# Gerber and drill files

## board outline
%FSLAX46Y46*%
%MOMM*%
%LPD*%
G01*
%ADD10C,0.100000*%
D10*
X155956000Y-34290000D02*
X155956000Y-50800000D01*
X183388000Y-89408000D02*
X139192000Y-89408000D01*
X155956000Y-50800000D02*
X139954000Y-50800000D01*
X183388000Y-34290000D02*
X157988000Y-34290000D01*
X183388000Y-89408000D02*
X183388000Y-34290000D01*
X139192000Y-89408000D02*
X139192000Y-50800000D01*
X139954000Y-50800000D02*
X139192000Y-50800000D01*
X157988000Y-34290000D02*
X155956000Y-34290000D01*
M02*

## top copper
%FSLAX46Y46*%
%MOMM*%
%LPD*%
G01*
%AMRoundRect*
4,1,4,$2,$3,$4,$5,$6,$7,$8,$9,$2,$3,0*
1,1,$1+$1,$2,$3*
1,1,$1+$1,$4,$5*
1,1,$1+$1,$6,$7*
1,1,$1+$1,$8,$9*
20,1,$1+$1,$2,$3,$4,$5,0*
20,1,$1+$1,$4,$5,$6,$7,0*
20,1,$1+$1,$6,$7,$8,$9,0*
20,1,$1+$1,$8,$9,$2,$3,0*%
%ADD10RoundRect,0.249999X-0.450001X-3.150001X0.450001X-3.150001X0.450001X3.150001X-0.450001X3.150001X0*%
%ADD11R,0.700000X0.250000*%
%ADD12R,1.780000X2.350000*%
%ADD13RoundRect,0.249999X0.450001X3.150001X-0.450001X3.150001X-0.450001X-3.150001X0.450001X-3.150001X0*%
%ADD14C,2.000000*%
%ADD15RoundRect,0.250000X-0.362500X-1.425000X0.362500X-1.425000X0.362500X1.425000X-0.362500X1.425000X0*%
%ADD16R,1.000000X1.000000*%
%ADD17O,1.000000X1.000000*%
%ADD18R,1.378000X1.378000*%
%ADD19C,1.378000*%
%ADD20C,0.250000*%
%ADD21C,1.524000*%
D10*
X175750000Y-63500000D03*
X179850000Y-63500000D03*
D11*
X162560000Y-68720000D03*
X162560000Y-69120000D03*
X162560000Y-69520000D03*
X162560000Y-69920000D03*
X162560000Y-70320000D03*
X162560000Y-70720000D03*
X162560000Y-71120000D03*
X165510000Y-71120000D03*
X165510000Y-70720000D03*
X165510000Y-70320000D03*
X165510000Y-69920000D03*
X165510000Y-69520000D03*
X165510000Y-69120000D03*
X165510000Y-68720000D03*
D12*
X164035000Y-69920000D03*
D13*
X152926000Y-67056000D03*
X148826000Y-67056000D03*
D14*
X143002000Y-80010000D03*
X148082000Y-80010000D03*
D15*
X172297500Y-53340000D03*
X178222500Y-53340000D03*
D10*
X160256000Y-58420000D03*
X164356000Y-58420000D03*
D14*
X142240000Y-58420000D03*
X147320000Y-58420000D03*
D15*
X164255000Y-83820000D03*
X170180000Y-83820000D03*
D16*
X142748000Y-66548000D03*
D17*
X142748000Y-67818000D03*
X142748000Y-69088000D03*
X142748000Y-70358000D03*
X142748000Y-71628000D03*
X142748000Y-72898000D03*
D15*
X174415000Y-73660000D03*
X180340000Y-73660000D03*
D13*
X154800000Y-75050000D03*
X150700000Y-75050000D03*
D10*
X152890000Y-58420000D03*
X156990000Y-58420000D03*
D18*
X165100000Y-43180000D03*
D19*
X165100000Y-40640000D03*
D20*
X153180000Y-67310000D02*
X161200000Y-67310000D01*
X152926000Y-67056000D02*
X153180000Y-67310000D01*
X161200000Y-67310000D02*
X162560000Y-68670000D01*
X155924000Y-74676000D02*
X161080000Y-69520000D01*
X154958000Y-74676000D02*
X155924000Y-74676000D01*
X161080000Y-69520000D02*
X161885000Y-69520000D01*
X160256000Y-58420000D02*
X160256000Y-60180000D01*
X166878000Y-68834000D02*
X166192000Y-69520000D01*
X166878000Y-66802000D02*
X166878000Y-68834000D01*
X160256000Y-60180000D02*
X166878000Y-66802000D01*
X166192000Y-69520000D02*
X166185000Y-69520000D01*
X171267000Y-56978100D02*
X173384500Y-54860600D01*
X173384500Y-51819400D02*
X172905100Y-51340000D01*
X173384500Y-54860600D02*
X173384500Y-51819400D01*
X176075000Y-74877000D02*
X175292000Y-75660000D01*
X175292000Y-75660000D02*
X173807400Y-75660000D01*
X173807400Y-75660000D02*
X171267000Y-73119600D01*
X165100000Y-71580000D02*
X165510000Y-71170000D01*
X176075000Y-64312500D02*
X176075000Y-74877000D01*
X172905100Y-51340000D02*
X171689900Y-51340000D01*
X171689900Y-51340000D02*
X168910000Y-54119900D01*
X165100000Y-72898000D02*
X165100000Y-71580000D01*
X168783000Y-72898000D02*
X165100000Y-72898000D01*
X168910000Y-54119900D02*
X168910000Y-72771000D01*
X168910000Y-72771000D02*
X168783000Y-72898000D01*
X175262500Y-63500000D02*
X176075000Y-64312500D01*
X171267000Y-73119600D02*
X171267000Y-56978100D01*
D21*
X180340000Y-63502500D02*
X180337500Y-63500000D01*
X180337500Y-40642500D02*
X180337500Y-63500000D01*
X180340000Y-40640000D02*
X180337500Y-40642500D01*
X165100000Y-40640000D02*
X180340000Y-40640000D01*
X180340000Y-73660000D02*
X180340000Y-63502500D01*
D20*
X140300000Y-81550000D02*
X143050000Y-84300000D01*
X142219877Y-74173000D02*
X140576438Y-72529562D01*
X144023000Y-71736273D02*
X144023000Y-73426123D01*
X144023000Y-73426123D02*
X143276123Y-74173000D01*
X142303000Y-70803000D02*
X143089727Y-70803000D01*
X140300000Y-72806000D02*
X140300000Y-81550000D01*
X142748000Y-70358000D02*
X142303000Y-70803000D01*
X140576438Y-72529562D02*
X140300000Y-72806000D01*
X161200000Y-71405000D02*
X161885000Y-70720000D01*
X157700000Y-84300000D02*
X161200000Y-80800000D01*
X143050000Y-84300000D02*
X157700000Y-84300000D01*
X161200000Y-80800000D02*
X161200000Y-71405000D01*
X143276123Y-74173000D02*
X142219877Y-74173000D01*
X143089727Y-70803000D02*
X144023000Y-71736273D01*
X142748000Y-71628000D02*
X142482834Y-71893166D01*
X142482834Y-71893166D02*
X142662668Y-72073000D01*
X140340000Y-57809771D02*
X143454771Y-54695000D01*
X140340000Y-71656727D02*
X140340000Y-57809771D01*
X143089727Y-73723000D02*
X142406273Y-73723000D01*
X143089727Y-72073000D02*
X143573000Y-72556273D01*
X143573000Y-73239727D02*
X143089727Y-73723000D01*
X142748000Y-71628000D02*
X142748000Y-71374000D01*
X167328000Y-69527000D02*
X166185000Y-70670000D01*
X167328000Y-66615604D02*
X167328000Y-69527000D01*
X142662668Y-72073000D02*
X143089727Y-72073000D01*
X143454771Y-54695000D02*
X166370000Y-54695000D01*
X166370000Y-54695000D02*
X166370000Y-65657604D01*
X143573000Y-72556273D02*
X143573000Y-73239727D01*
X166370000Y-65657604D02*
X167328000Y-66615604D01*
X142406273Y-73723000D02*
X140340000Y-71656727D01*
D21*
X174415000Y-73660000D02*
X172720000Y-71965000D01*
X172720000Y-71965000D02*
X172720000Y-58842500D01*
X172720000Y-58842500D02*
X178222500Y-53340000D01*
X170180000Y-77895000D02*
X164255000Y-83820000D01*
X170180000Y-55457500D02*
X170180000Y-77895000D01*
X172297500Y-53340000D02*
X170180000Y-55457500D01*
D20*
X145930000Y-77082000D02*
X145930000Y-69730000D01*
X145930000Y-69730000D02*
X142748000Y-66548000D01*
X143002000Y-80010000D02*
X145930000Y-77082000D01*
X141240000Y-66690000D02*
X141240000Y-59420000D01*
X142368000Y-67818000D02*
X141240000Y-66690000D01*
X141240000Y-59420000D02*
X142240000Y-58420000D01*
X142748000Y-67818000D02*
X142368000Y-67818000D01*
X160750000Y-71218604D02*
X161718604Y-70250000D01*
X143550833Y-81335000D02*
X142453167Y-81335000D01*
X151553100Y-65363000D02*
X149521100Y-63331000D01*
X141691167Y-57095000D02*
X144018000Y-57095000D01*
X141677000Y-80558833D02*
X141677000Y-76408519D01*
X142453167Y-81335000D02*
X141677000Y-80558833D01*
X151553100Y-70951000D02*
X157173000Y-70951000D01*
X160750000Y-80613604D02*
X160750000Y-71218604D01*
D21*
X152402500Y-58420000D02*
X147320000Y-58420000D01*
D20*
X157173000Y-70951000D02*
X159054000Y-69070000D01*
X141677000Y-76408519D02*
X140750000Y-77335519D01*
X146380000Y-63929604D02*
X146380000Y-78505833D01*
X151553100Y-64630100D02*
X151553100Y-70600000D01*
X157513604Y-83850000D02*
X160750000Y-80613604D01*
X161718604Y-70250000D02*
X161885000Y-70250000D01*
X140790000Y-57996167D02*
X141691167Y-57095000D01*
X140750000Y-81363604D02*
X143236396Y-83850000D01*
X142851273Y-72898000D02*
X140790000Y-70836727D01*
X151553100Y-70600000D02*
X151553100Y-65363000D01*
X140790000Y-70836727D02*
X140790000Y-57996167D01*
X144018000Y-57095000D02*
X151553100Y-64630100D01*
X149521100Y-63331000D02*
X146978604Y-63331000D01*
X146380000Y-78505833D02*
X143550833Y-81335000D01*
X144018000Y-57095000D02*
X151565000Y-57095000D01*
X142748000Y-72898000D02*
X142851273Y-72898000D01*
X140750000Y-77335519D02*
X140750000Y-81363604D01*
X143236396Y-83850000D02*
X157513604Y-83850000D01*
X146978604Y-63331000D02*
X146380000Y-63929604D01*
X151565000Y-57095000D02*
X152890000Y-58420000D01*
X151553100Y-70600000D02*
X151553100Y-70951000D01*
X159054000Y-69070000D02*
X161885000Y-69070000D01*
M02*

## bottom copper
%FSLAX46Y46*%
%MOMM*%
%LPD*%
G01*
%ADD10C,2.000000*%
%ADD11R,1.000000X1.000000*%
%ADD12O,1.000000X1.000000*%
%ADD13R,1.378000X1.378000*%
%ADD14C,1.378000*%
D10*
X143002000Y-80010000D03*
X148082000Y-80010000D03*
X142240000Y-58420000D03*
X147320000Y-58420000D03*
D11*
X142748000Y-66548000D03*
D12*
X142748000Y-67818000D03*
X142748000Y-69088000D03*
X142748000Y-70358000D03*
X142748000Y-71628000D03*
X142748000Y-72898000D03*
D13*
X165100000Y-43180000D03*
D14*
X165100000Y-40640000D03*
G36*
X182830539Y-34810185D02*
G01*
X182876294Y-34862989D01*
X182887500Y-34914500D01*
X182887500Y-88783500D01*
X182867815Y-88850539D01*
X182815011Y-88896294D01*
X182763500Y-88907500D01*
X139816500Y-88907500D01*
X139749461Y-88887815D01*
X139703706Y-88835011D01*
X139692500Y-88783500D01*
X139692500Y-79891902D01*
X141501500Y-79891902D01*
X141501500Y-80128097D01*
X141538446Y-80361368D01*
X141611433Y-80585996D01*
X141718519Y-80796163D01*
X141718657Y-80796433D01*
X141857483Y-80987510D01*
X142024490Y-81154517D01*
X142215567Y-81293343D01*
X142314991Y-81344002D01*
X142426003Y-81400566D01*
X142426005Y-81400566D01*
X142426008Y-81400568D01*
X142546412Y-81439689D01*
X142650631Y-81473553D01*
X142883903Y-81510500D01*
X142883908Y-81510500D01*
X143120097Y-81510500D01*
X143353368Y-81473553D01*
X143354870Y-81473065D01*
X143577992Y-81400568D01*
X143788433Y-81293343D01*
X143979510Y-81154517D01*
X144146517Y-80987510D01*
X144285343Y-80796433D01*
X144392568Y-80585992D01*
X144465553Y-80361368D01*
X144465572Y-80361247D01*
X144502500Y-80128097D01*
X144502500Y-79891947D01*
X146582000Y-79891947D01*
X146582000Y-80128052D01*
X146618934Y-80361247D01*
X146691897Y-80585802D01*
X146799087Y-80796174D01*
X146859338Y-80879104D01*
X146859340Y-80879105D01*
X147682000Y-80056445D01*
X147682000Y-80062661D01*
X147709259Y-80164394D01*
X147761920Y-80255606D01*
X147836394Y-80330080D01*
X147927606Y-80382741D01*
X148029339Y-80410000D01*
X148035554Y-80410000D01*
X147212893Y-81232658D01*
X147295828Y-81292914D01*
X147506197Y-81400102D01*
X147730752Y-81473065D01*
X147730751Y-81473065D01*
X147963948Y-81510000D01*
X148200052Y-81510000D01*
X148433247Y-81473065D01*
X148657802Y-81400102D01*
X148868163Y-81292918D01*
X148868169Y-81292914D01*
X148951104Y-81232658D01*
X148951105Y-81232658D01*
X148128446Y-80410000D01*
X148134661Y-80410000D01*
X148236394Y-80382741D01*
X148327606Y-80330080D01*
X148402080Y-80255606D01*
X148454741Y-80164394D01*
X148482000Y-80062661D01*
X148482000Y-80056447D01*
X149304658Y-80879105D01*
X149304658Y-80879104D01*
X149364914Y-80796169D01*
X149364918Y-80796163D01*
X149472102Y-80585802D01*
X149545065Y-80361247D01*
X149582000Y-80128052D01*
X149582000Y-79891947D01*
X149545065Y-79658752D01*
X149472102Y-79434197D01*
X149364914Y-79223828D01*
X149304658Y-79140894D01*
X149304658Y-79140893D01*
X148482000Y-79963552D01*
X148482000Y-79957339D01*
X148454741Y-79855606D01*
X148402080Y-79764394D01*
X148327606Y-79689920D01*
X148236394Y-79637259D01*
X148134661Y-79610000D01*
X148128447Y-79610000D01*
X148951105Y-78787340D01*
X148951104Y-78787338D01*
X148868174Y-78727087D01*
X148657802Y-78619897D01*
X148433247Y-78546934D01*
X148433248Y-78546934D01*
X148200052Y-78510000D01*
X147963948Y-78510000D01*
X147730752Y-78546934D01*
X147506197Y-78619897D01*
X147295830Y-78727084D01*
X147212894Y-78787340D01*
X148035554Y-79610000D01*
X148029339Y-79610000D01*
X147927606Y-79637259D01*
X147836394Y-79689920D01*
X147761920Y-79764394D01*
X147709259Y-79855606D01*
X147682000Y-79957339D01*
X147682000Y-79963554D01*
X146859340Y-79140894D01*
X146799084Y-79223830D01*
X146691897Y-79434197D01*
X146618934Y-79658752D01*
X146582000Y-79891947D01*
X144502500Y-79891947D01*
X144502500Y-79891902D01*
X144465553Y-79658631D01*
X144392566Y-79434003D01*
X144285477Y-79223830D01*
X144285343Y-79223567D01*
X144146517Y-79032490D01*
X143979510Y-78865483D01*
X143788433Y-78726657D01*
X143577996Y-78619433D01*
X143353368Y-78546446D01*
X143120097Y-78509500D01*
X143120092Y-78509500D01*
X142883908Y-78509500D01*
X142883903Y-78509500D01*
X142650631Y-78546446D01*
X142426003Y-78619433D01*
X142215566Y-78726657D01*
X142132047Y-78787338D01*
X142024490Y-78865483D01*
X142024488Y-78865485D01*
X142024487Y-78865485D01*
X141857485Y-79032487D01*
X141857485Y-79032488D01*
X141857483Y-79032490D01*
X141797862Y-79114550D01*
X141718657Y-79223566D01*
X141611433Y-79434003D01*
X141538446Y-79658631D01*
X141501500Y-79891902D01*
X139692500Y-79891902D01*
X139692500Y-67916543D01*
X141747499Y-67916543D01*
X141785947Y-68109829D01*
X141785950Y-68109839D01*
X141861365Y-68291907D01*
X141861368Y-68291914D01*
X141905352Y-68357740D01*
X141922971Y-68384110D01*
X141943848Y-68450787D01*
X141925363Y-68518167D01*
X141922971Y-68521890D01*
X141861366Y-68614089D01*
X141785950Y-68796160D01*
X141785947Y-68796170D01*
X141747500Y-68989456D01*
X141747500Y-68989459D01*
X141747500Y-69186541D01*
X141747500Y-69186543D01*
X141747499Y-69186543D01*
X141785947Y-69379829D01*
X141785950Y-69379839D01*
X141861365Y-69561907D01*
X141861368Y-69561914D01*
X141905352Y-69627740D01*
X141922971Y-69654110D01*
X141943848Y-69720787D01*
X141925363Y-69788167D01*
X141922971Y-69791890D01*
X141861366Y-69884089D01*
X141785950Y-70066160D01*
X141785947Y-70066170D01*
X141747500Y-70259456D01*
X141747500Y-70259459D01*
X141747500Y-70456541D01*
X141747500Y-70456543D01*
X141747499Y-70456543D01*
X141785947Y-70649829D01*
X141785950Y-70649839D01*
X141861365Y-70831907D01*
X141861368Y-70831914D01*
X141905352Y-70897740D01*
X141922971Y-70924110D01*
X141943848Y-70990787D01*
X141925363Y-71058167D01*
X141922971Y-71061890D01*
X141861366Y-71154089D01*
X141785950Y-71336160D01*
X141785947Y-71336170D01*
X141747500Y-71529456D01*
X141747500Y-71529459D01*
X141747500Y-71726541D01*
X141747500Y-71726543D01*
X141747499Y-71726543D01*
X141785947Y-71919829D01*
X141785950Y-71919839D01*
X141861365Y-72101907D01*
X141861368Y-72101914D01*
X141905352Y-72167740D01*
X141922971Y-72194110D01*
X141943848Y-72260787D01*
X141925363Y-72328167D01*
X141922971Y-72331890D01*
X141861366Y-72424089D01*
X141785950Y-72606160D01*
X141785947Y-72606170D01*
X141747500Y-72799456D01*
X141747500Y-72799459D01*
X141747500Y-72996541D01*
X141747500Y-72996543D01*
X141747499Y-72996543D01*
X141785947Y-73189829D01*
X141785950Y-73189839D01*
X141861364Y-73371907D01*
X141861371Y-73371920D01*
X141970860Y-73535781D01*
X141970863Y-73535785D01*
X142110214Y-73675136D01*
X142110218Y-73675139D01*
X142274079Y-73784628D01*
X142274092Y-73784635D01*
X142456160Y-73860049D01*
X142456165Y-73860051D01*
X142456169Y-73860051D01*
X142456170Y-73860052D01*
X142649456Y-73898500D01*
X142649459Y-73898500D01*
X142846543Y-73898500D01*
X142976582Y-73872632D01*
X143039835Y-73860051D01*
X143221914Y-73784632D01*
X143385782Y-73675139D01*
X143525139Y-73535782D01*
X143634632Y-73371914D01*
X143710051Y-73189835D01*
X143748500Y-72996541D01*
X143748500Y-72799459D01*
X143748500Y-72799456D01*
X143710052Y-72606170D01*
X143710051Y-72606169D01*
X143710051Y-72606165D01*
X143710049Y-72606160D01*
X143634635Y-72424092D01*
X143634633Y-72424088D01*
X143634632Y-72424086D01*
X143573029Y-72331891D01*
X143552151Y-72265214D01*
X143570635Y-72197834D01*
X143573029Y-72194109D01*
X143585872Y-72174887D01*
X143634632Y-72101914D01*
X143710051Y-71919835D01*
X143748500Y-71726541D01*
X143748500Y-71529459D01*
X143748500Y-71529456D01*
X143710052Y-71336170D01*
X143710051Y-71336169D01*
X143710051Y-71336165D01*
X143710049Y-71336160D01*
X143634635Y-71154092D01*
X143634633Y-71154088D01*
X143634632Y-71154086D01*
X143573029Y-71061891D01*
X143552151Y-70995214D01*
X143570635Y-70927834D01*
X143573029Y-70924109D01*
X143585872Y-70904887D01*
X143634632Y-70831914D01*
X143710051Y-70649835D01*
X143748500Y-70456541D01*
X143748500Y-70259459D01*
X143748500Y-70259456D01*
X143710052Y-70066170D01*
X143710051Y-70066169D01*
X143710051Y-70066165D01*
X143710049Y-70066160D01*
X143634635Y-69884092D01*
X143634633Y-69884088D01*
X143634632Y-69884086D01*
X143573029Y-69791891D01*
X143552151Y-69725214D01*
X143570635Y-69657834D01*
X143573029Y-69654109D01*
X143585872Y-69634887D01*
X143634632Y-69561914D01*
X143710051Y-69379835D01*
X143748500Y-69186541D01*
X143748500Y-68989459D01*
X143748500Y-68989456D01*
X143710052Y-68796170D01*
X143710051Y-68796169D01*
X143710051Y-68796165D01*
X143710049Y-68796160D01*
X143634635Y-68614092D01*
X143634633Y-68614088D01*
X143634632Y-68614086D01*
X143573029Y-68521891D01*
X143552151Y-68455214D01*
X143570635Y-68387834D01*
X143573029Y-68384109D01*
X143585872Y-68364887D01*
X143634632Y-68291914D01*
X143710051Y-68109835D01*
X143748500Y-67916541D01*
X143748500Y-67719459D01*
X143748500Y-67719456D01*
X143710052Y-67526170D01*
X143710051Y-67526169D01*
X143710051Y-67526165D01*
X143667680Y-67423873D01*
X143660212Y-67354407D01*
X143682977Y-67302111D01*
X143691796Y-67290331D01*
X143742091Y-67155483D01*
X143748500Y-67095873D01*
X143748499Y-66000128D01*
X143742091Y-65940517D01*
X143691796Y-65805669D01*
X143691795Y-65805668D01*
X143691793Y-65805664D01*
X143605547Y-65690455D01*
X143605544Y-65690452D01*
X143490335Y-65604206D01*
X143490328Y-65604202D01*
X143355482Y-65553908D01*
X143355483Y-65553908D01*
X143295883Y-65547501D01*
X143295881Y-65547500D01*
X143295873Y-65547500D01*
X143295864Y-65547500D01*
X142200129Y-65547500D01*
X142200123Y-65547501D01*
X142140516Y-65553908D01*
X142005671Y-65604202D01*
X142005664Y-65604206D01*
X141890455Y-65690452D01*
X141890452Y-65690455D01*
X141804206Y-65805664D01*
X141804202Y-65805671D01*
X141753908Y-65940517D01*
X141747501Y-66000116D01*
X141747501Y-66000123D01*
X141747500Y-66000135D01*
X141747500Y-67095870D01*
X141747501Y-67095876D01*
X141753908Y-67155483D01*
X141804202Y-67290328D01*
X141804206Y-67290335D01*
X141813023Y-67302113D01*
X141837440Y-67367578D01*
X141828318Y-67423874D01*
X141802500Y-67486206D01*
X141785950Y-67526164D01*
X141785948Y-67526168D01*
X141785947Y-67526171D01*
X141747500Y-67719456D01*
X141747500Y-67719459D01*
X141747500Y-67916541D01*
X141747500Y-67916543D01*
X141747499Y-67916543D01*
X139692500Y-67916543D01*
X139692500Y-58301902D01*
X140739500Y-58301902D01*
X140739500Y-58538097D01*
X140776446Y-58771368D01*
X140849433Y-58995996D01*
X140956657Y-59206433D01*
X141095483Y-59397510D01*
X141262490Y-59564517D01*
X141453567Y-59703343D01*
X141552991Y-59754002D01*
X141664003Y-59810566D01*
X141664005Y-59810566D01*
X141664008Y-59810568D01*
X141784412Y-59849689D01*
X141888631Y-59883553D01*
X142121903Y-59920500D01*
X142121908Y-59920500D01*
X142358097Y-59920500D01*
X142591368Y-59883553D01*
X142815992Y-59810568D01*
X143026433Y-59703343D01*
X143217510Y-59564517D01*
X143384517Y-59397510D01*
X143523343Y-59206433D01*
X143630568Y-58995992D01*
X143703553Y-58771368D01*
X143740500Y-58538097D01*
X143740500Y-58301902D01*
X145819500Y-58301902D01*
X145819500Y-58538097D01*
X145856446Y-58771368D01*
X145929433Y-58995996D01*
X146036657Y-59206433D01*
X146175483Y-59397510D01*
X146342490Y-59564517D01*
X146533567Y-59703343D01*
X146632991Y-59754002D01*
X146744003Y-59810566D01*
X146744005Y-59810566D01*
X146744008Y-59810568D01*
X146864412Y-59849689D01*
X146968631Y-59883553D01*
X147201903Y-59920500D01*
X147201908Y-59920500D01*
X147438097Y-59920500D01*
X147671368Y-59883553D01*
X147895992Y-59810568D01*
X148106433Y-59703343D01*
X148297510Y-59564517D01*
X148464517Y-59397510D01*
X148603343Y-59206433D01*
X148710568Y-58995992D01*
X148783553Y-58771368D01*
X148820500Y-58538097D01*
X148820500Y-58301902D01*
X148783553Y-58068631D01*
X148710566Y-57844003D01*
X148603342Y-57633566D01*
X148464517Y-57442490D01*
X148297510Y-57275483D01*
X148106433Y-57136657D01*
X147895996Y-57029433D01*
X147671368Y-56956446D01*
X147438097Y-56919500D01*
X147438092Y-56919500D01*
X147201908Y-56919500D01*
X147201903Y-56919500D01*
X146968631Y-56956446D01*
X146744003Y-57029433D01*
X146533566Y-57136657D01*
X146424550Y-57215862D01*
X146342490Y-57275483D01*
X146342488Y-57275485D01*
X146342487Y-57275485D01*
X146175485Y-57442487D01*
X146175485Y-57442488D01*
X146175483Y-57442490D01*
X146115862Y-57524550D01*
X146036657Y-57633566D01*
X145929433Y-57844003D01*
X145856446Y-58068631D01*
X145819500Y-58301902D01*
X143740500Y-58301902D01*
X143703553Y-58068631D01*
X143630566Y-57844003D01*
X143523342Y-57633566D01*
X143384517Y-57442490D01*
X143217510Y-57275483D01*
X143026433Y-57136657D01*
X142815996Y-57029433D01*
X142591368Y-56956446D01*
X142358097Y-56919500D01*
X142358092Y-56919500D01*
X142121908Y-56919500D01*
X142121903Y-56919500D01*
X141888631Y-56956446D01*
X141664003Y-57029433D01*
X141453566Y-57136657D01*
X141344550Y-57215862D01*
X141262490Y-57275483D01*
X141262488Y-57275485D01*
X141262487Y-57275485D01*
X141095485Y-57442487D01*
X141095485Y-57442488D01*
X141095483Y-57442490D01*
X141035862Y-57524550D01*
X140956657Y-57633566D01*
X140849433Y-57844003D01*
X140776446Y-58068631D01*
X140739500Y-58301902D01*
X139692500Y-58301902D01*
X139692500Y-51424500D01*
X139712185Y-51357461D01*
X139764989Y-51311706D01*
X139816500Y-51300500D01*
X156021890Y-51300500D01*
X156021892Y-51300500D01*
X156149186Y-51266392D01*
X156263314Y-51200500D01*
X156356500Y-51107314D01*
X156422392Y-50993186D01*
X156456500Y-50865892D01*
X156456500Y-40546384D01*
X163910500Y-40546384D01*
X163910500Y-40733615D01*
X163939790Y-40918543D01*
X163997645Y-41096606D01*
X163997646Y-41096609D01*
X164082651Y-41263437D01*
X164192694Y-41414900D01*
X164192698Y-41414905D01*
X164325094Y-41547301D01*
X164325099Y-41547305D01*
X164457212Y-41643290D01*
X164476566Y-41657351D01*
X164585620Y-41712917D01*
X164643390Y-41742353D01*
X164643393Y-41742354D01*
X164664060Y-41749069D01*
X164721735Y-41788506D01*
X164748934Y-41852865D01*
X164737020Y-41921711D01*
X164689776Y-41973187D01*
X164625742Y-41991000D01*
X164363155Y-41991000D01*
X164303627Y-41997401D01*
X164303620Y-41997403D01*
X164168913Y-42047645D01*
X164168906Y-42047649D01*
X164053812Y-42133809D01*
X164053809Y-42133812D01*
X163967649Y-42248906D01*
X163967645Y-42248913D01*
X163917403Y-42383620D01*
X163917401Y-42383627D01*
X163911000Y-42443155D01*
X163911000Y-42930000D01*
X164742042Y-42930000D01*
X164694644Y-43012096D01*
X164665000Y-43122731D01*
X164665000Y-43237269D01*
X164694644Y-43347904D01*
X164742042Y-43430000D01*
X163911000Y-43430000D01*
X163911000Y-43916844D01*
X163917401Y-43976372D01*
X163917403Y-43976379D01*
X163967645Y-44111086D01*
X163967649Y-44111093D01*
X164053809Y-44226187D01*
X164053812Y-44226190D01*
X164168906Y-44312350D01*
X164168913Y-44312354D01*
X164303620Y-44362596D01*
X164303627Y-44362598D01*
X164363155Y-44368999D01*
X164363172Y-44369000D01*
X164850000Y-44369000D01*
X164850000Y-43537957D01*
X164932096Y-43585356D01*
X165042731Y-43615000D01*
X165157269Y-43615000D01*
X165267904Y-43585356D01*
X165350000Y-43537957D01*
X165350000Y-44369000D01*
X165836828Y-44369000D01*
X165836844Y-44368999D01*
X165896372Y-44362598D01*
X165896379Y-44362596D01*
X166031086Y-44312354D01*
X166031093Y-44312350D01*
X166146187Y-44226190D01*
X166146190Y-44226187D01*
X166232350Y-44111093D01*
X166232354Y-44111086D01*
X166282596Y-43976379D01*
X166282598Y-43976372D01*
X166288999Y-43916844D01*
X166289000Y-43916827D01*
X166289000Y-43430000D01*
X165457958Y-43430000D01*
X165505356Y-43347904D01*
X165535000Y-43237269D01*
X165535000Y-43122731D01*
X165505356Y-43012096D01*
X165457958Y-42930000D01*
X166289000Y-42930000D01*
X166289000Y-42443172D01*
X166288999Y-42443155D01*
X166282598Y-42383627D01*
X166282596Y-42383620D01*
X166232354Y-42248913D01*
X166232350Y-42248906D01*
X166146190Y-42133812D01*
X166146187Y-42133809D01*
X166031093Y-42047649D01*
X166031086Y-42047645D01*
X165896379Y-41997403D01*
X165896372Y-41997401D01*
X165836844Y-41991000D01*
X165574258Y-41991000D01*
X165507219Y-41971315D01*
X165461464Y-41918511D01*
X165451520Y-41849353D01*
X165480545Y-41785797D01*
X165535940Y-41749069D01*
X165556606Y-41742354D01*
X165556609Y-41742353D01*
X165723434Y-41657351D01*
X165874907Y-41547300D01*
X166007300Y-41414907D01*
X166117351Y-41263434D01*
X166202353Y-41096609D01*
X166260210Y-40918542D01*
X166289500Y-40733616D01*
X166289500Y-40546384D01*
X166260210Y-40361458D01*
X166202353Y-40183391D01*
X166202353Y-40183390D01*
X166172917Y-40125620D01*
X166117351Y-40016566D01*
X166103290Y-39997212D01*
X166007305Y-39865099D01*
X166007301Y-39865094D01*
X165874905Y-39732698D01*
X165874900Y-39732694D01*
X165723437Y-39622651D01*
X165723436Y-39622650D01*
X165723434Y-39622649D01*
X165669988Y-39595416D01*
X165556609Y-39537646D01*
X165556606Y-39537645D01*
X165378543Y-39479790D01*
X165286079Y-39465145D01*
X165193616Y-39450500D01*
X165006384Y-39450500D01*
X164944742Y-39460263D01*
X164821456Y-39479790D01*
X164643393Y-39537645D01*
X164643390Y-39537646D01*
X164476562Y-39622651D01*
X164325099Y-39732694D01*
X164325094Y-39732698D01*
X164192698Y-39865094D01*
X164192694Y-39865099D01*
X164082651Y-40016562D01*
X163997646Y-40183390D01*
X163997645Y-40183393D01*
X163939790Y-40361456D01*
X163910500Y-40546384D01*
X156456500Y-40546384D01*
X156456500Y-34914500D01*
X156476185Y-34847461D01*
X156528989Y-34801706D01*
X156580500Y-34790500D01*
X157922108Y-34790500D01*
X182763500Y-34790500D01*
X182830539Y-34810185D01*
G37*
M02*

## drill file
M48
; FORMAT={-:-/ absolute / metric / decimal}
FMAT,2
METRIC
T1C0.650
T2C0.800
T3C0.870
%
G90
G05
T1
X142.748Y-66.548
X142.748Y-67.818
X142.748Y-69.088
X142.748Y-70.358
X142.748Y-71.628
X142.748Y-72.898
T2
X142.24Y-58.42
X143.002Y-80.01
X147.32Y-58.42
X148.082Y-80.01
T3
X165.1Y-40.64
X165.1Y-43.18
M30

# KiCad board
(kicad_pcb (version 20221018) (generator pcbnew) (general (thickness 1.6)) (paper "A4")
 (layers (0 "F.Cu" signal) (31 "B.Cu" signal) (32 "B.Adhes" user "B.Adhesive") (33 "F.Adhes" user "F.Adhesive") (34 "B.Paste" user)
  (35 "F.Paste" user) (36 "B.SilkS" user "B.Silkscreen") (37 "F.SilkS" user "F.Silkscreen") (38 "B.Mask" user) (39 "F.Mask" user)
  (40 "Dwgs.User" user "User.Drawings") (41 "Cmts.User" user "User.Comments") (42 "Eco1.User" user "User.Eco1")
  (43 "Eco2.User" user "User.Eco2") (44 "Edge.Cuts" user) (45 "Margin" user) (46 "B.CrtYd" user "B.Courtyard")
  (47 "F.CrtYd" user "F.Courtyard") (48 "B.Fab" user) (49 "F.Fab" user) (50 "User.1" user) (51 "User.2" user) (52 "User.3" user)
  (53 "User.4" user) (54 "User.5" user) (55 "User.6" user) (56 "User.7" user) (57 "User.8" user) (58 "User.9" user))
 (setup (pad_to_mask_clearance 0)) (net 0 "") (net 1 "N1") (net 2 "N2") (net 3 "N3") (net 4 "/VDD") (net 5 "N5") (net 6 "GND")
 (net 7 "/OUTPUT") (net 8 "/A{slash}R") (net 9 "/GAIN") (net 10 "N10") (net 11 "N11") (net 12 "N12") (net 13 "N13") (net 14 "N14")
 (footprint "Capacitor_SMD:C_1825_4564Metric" (layer "F.Cu") (at 177.8 63.5)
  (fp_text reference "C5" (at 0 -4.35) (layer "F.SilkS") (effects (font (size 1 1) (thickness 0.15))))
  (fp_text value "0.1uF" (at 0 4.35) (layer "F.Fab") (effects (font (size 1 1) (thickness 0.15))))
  (pad "1" smd roundrect (at -2.05 0) (size 1.4 6.8) (layers "F.Cu" "F.Paste" "F.Mask") (roundrect_rratio 0.178571) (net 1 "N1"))
  (pad "2" smd roundrect (at 2.05 0) (size 1.4 6.8) (layers "F.Cu" "F.Paste" "F.Mask") (roundrect_rratio 0.178571) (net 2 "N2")))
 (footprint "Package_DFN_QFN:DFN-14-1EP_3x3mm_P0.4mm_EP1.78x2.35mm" (layer "F.Cu") (at 164.035 69.92)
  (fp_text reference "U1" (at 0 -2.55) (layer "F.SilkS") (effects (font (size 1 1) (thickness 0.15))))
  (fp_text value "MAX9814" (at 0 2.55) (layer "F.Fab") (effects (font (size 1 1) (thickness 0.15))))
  (pad "" smd rect (at -0.445 -0.5875) (size 0.7 0.97) (layers "F.Paste"))
  (pad "" smd rect (at -0.445 0.5875) (size 0.7 0.97) (layers "F.Paste"))
  (pad "" smd rect (at 0.45 -0.5875) (size 0.7 0.97) (layers "F.Paste"))
  (pad "" smd rect (at 0.45 0.5875) (size 0.7 0.97) (layers "F.Paste"))
  (pad "1" smd rect (at -1.475 -1.2) (size 0.7 0.25) (layers "F.Cu" "F.Paste" "F.Mask") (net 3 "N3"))
  (pad "2" smd rect (at -1.475 -0.8) (size 0.7 0.25) (layers "F.Cu" "F.Paste" "F.Mask") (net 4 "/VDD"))
  (pad "3" smd rect (at -1.475 -0.4) (size 0.7 0.25) (layers "F.Cu" "F.Paste" "F.Mask") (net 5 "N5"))
  (pad "4" smd rect (at -1.475 0) (size 0.7 0.25) (layers "F.Cu" "F.Paste" "F.Mask") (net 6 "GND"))
  (pad "5" smd rect (at -1.475 0.4) (size 0.7 0.25) (layers "F.Cu" "F.Paste" "F.Mask") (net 4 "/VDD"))
  (pad "6" smd rect (at -1.475 0.8) (size 0.7 0.25) (layers "F.Cu" "F.Paste" "F.Mask") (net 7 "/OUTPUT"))
  (pad "7" smd rect (at -1.475 1.2) (size 0.7 0.25) (layers "F.Cu" "F.Paste" "F.Mask") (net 6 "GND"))
  (pad "8" smd rect (at 1.475 1.2) (size 0.7 0.25) (layers "F.Cu" "F.Paste" "F.Mask") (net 1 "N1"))
  (pad "9" smd rect (at 1.475 0.8) (size 0.7 0.25) (layers "F.Cu" "F.Paste" "F.Mask") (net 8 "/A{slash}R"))
  (pad "10" smd rect (at 1.475 0.4) (size 0.7 0.25) (layers "F.Cu" "F.Paste" "F.Mask") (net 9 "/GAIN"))
  (pad "11" smd rect (at 1.475 0) (size 0.7 0.25) (layers "F.Cu" "F.Paste" "F.Mask") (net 6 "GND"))
  (pad "12" smd rect (at 1.475 -0.4) (size 0.7 0.25) (layers "F.Cu" "F.Paste" "F.Mask") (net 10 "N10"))
  (pad "13" smd rect (at 1.475 -0.8) (size 0.7 0.25) (layers "F.Cu" "F.Paste" "F.Mask") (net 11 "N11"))
  (pad "14" smd rect (at 1.475 -1.2) (size 0.7 0.25) (layers "F.Cu" "F.Paste" "F.Mask") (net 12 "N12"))
  (pad "15" smd rect (at 0 0) (size 1.78 2.35) (layers "F.Cu" "F.Mask") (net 6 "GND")))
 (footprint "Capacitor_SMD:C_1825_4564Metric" (layer "F.Cu") (at 150.876 67.056 180)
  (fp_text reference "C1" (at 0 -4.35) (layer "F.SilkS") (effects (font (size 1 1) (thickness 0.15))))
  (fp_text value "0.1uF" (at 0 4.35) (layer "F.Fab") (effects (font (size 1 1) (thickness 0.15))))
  (pad "1" smd roundrect (at -2.05 0 180) (size 1.4 6.8) (layers "F.Cu" "F.Paste" "F.Mask") (roundrect_rratio 0.178571) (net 3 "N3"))
  (pad "2" smd roundrect (at 2.05 0 180) (size 1.4 6.8) (layers "F.Cu" "F.Paste" "F.Mask") (roundrect_rratio 0.178571) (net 6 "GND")))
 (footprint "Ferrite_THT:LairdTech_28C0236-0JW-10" (layer "F.Cu") (at 143.002 80.01)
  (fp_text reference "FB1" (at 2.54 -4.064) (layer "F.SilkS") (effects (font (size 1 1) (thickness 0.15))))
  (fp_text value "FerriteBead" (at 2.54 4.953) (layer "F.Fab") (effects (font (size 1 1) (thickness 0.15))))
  (pad "1" thru_hole circle (at 0 0) (size 2 2) (drill 0.8) (layers "*.Cu" "*.Mask") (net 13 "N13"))
  (pad "2" thru_hole circle (at 5.08 0) (size 2 2) (drill 0.8) (layers "*.Cu" "*.Mask") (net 6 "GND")))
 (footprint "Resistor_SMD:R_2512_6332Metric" (layer "F.Cu") (at 175.26 53.34)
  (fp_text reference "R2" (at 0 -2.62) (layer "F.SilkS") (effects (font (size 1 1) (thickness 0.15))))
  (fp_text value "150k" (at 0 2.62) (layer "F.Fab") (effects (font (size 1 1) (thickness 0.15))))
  (pad "1" smd roundrect (at -2.9625 0) (size 1.225 3.35) (layers "F.Cu" "F.Paste" "F.Mask") (roundrect_rratio 0.204082) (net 12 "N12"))
  (pad "2" smd roundrect (at 2.9625 0) (size 1.225 3.35) (layers "F.Cu" "F.Paste" "F.Mask") (roundrect_rratio 0.204082) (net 11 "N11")))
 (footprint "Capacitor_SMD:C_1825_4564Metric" (layer "F.Cu") (at 162.306 58.42)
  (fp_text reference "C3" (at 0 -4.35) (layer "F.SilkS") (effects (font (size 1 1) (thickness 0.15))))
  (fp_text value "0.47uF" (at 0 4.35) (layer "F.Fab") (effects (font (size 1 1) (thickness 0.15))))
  (pad "1" smd roundrect (at -2.05 0) (size 1.4 6.8) (layers "F.Cu" "F.Paste" "F.Mask") (roundrect_rratio 0.178571) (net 10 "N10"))
  (pad "2" smd roundrect (at 2.05 0) (size 1.4 6.8) (layers "F.Cu" "F.Paste" "F.Mask") (roundrect_rratio 0.178571) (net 6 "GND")))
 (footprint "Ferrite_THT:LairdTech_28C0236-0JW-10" (layer "F.Cu") (at 142.24 58.42)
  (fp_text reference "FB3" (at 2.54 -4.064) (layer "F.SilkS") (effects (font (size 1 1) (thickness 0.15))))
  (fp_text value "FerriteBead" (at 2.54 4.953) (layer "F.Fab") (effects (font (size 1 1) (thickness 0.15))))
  (pad "1" thru_hole circle (at 0 0) (size 2 2) (drill 0.8) (layers "*.Cu" "*.Mask") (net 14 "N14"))
  (pad "2" thru_hole circle (at 5.08 0) (size 2 2) (drill 0.8) (layers "*.Cu" "*.Mask") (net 4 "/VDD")))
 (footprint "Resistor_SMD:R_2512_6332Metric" (layer "F.Cu") (at 167.2175 83.82)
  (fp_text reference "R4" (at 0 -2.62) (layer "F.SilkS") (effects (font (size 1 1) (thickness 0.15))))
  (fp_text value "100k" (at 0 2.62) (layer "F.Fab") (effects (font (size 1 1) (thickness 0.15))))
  (pad "1" smd roundrect (at -2.9625 0) (size 1.225 3.35) (layers "F.Cu" "F.Paste" "F.Mask") (roundrect_rratio 0.204082) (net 12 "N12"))
  (pad "2" smd roundrect (at 2.9625 0) (size 1.225 3.35) (layers "F.Cu" "F.Paste" "F.Mask") (roundrect_rratio 0.204082) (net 6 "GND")))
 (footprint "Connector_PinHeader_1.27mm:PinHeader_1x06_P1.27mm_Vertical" (layer "F.Cu") (at 142.748 66.548)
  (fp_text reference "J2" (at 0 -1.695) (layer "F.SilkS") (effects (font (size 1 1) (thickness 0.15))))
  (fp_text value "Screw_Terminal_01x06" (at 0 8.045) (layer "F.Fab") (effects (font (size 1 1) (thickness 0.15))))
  (pad "1" thru_hole rect (at 0 0) (size 1 1) (drill 0.65) (layers "*.Cu" "*.Mask") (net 13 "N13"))
  (pad "2" thru_hole oval (at 0 1.27) (size 1 1) (drill 0.65) (layers "*.Cu" "*.Mask") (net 14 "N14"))
  (pad "3" thru_hole oval (at 0 2.54) (size 1 1) (drill 0.65) (layers "*.Cu" "*.Mask") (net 9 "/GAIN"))
  (pad "4" thru_hole oval (at 0 3.81) (size 1 1) (drill 0.65) (layers "*.Cu" "*.Mask") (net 7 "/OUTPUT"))
  (pad "5" thru_hole oval (at 0 5.08) (size 1 1) (drill 0.65) (layers "*.Cu" "*.Mask") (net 8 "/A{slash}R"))
  (pad "6" thru_hole oval (at 0 6.35) (size 1 1) (drill 0.65) (layers "*.Cu" "*.Mask") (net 4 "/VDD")))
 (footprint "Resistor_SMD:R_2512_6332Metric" (layer "F.Cu") (at 177.3775 73.66)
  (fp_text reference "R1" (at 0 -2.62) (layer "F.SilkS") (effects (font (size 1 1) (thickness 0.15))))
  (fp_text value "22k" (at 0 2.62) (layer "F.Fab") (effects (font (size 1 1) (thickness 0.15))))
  (pad "1" smd roundrect (at -2.9625 0) (size 1.225 3.35) (layers "F.Cu" "F.Paste" "F.Mask") (roundrect_rratio 0.204082) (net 11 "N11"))
  (pad "2" smd roundrect (at 2.9625 0) (size 1.225 3.35) (layers "F.Cu" "F.Paste" "F.Mask") (roundrect_rratio 0.204082) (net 2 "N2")))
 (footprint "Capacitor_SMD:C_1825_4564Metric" (layer "F.Cu") (at 152.75 75.05 180)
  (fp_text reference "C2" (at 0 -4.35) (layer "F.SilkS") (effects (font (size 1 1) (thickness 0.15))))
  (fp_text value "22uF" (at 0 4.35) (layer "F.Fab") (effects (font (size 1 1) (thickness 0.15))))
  (pad "1" smd roundrect (at -2.05 0 180) (size 1.4 6.8) (layers "F.Cu" "F.Paste" "F.Mask") (roundrect_rratio 0.178571) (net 5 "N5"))
  (pad "2" smd roundrect (at 2.05 0 180) (size 1.4 6.8) (layers "F.Cu" "F.Paste" "F.Mask") (roundrect_rratio 0.178571) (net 6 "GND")))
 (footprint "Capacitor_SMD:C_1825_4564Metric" (layer "F.Cu") (at 154.94 58.42)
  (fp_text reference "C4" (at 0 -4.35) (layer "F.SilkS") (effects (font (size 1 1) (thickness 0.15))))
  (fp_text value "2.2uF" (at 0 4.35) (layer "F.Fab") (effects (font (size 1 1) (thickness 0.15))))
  (pad "1" smd roundrect (at -2.05 0) (size 1.4 6.8) (layers "F.Cu" "F.Paste" "F.Mask") (roundrect_rratio 0.178571) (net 4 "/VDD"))
  (pad "2" smd roundrect (at 2.05 0) (size 1.4 6.8) (layers "F.Cu" "F.Paste" "F.Mask") (roundrect_rratio 0.178571) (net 6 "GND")))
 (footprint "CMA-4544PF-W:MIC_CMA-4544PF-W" (layer "F.Cu") (at 163.1 41.91)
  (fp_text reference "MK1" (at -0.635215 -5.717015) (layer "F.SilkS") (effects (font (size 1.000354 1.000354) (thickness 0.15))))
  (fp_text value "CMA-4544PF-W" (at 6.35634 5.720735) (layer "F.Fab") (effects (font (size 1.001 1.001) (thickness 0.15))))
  (pad "1" thru_hole rect (at 2 1.27) (size 1.378 1.378) (drill 0.87) (layers "*.Cu" "*.Mask") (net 6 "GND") (solder_mask_margin 0.102))
  (pad "2" thru_hole circle (at 2 -1.27) (size 1.378 1.378) (drill 0.87) (layers "*.Cu" "*.Mask") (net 2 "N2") (solder_mask_margin 0.102)))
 (gr_line (start 155.956 34.29) (end 155.956 50.8) (stroke (width 0.1) (type default)) (layer "Edge.Cuts"))
 (gr_line (start 183.388 89.408) (end 139.192 89.408) (stroke (width 0.1) (type default)) (layer "Edge.Cuts"))
 (gr_line (start 155.956 50.8) (end 139.954 50.8) (stroke (width 0.1) (type default)) (layer "Edge.Cuts"))
 (gr_line (start 183.388 34.29) (end 157.988 34.29) (stroke (width 0.1) (type default)) (layer "Edge.Cuts"))
 (gr_line (start 183.388 89.408) (end 183.388 34.29) (stroke (width 0.1) (type default)) (layer "Edge.Cuts"))
 (gr_line (start 139.192 89.408) (end 139.192 50.8) (stroke (width 0.1) (type default)) (layer "Edge.Cuts"))
 (gr_line (start 139.954 50.8) (end 139.192 50.8) (stroke (width 0.1) (type default)) (layer "Edge.Cuts"))
 (gr_line (start 157.988 34.29) (end 155.956 34.29) (stroke (width 0.1) (type default)) (layer "Edge.Cuts"))
 (segment (start 153.18 67.31) (end 161.2 67.31) (width 0.25) (layer "F.Cu") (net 3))
 (segment (start 152.926 67.056) (end 153.18 67.31) (width 0.25) (layer "F.Cu") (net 3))
 (segment (start 161.2 67.31) (end 162.56 68.67) (width 0.25) (layer "F.Cu") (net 3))
 (segment (start 155.924 74.676) (end 161.08 69.52) (width 0.25) (layer "F.Cu") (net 5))
 (segment (start 154.958 74.676) (end 155.924 74.676) (width 0.25) (layer "F.Cu") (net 5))
 (segment (start 161.08 69.52) (end 161.885 69.52) (width 0.25) (layer "F.Cu") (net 5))
 (segment (start 160.256 58.42) (end 160.256 60.18) (width 0.25) (layer "F.Cu") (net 10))
 (segment (start 166.878 68.834) (end 166.192 69.52) (width 0.25) (layer "F.Cu") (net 10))
 (segment (start 166.878 66.802) (end 166.878 68.834) (width 0.25) (layer "F.Cu") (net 10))
 (segment (start 160.256 60.18) (end 166.878 66.802) (width 0.25) (layer "F.Cu") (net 10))
 (segment (start 166.192 69.52) (end 166.185 69.52) (width 0.25) (layer "F.Cu") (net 10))
 (segment (start 171.267 56.9781) (end 173.3845 54.8606) (width 0.25) (layer "F.Cu") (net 1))
 (segment (start 173.3845 51.8194) (end 172.9051 51.34) (width 0.25) (layer "F.Cu") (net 1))
 (segment (start 173.3845 54.8606) (end 173.3845 51.8194) (width 0.25) (layer "F.Cu") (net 1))
 (segment (start 176.075 74.877) (end 175.292 75.66) (width 0.25) (layer "F.Cu") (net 1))
 (segment (start 175.292 75.66) (end 173.8074 75.66) (width 0.25) (layer "F.Cu") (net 1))
 (segment (start 173.8074 75.66) (end 171.267 73.1196) (width 0.25) (layer "F.Cu") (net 1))
 (segment (start 165.1 71.58) (end 165.51 71.17) (width 0.25) (layer "F.Cu") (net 1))
 (segment (start 176.075 64.3125) (end 176.075 74.877) (width 0.25) (layer "F.Cu") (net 1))
 (segment (start 172.9051 51.34) (end 171.6899 51.34) (width 0.25) (layer "F.Cu") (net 1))
 (segment (start 171.6899 51.34) (end 168.91 54.1199) (width 0.25) (layer "F.Cu") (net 1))
 (segment (start 165.1 72.898) (end 165.1 71.58) (width 0.25) (layer "F.Cu") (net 1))
 (segment (start 168.783 72.898) (end 165.1 72.898) (width 0.25) (layer "F.Cu") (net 1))
 (segment (start 168.91 54.1199) (end 168.91 72.771) (width 0.25) (layer "F.Cu") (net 1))
 (segment (start 168.91 72.771) (end 168.783 72.898) (width 0.25) (layer "F.Cu") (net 1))
 (segment (start 175.2625 63.5) (end 176.075 64.3125) (width 0.25) (layer "F.Cu") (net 1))
 (segment (start 171.267 73.1196) (end 171.267 56.9781) (width 0.25) (layer "F.Cu") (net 1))
 (segment (start 180.34 63.5025) (end 180.3375 63.5) (width 1.524) (layer "F.Cu") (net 2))
 (segment (start 180.3375 40.6425) (end 180.3375 63.5) (width 1.524) (layer "F.Cu") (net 2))
 (segment (start 180.34 40.64) (end 180.3375 40.6425) (width 1.524) (layer "F.Cu") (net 2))
 (segment (start 165.1 40.64) (end 180.34 40.64) (width 1.524) (layer "F.Cu") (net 2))
 (segment (start 180.34 73.66) (end 180.34 63.5025) (width 1.524) (layer "F.Cu") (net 2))
 (segment (start 140.3 81.55) (end 143.05 84.3) (width 0.25) (layer "F.Cu") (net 7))
 (segment (start 142.219877 74.173) (end 140.576438 72.529562) (width 0.25) (layer "F.Cu") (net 7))
 (segment (start 144.023 71.736273) (end 144.023 73.426123) (width 0.25) (layer "F.Cu") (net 7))
 (segment (start 144.023 73.426123) (end 143.276123 74.173) (width 0.25) (layer "F.Cu") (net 7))
 (segment (start 142.303 70.803) (end 143.089727 70.803) (width 0.25) (layer "F.Cu") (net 7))
 (segment (start 140.3 72.806) (end 140.3 81.55) (width 0.25) (layer "F.Cu") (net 7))
 (segment (start 142.748 70.358) (end 142.303 70.803) (width 0.25) (layer "F.Cu") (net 7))
 (segment (start 140.576438 72.529562) (end 140.3 72.806) (width 0.25) (layer "F.Cu") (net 7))
 (segment (start 161.2 71.405) (end 161.885 70.72) (width 0.25) (layer "F.Cu") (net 7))
 (segment (start 157.7 84.3) (end 161.2 80.8) (width 0.25) (layer "F.Cu") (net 7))
 (segment (start 143.05 84.3) (end 157.7 84.3) (width 0.25) (layer "F.Cu") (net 7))
 (segment (start 161.2 80.8) (end 161.2 71.405) (width 0.25) (layer "F.Cu") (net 7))
 (segment (start 143.276123 74.173) (end 142.219877 74.173) (width 0.25) (layer "F.Cu") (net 7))
 (segment (start 143.089727 70.803) (end 144.023 71.736273) (width 0.25) (layer "F.Cu") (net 7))
 (segment (start 142.748 71.628) (end 142.482834 71.893166) (width 0.25) (layer "F.Cu") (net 8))
 (segment (start 142.482834 71.893166) (end 142.662668 72.073) (width 0.25) (layer "F.Cu") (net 8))
 (segment (start 140.34 57.809771) (end 143.454771 54.695) (width 0.25) (layer "F.Cu") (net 8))
 (segment (start 140.34 71.656727) (end 140.34 57.809771) (width 0.25) (layer "F.Cu") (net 8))
 (segment (start 143.089727 73.723) (end 142.406273 73.723) (width 0.25) (layer "F.Cu") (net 8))
 (segment (start 143.089727 72.073) (end 143.573 72.556273) (width 0.25) (layer "F.Cu") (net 8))
 (segment (start 143.573 73.239727) (end 143.089727 73.723) (width 0.25) (layer "F.Cu") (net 8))
 (segment (start 142.748 71.628) (end 142.748 71.374) (width 0.25) (layer "F.Cu") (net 8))
 (segment (start 167.328 69.527) (end 166.185 70.67) (width 0.25) (layer "F.Cu") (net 8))
 (segment (start 167.328 66.615604) (end 167.328 69.527) (width 0.25) (layer "F.Cu") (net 8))
 (segment (start 142.662668 72.073) (end 143.089727 72.073) (width 0.25) (layer "F.Cu") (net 8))
 (segment (start 143.454771 54.695) (end 166.37 54.695) (width 0.25) (layer "F.Cu") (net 8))
 (segment (start 166.37 54.695) (end 166.37 65.657604) (width 0.25) (layer "F.Cu") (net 8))
 (segment (start 143.573 72.556273) (end 143.573 73.239727) (width 0.25) (layer "F.Cu") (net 8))
 (segment (start 166.37 65.657604) (end 167.328 66.615604) (width 0.25) (layer "F.Cu") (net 8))
 (segment (start 142.406273 73.723) (end 140.34 71.656727) (width 0.25) (layer "F.Cu") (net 8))
 (segment (start 174.415 73.66) (end 172.72 71.965) (width 1.524) (layer "F.Cu") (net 11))
 (segment (start 172.72 71.965) (end 172.72 58.8425) (width 1.524) (layer "F.Cu") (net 11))
 (segment (start 172.72 58.8425) (end 178.2225 53.34) (width 1.524) (layer "F.Cu") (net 11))
 (segment (start 170.18 77.895) (end 164.255 83.82) (width 1.524) (layer "F.Cu") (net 12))
 (segment (start 170.18 55.4575) (end 170.18 77.895) (width 1.524) (layer "F.Cu") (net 12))
 (segment (start 172.2975 53.34) (end 170.18 55.4575) (width 1.524) (layer "F.Cu") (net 12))
 (segment (start 145.93 77.082) (end 145.93 69.73) (width 0.25) (layer "F.Cu") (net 13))
 (segment (start 145.93 69.73) (end 142.748 66.548) (width 0.25) (layer "F.Cu") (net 13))
 (segment (start 143.002 80.01) (end 145.93 77.082) (width 0.25) (layer "F.Cu") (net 13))
 (segment (start 141.24 66.69) (end 141.24 59.42) (width 0.25) (layer "F.Cu") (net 14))
 (segment (start 142.368 67.818) (end 141.24 66.69) (width 0.25) (layer "F.Cu") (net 14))
 (segment (start 141.24 59.42) (end 142.24 58.42) (width 0.25) (layer "F.Cu") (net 14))
 (segment (start 142.748 67.818) (end 142.368 67.818) (width 0.25) (layer "F.Cu") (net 14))
 (segment (start 160.75 71.218604) (end 161.718604 70.25) (width 0.25) (layer "F.Cu") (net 4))
 (segment (start 143.550833 81.335) (end 142.453167 81.335) (width 0.25) (layer "F.Cu") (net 4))
 (segment (start 151.5531 65.363) (end 149.5211 63.331) (width 0.25) (layer "F.Cu") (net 4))
 (segment (start 141.691167 57.095) (end 144.018 57.095) (width 0.25) (layer "F.Cu") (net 4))
 (segment (start 141.677 80.558833) (end 141.677 76.408519) (width 0.25) (layer "F.Cu") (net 4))
 (segment (start 142.453167 81.335) (end 141.677 80.558833) (width 0.25) (layer "F.Cu") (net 4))
 (segment (start 151.5531 70.951) (end 157.173 70.951) (width 0.25) (layer "F.Cu") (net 4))
 (segment (start 160.75 80.613604) (end 160.75 71.218604) (width 0.25) (layer "F.Cu") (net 4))
 (segment (start 152.4025 58.42) (end 147.32 58.42) (width 1.524) (layer "F.Cu") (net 4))
 (segment (start 157.173 70.951) (end 159.054 69.07) (width 0.25) (layer "F.Cu") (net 4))
 (segment (start 141.677 76.408519) (end 140.75 77.335519) (width 0.25) (layer "F.Cu") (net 4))
 (segment (start 146.38 63.929604) (end 146.38 78.505833) (width 0.25) (layer "F.Cu") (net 4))
 (segment (start 151.5531 64.6301) (end 151.5531 70.6) (width 0.25) (layer "F.Cu") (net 4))
 (segment (start 157.513604 83.85) (end 160.75 80.613604) (width 0.25) (layer "F.Cu") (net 4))
 (segment (start 161.718604 70.25) (end 161.885 70.25) (width 0.25) (layer "F.Cu") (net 4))
 (segment (start 140.79 57.996167) (end 141.691167 57.095) (width 0.25) (layer "F.Cu") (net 4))
 (segment (start 140.75 81.363604) (end 143.236396 83.85) (width 0.25) (layer "F.Cu") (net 4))
 (segment (start 142.851273 72.898) (end 140.79 70.836727) (width 0.25) (layer "F.Cu") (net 4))
 (segment (start 151.5531 70.6) (end 151.5531 65.363) (width 0.25) (layer "F.Cu") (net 4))
 (segment (start 140.79 70.836727) (end 140.79 57.996167) (width 0.25) (layer "F.Cu") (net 4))
 (segment (start 144.018 57.095) (end 151.5531 64.6301) (width 0.25) (layer "F.Cu") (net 4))
 (segment (start 149.5211 63.331) (end 146.978604 63.331) (width 0.25) (layer "F.Cu") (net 4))
 (segment (start 146.38 78.505833) (end 143.550833 81.335) (width 0.25) (layer "F.Cu") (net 4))
 (segment (start 144.018 57.095) (end 151.565 57.095) (width 0.25) (layer "F.Cu") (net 4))
 (segment (start 142.748 72.898) (end 142.851273 72.898) (width 0.25) (layer "F.Cu") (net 4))
 (segment (start 140.75 77.335519) (end 140.75 81.363604) (width 0.25) (layer "F.Cu") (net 4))
 (segment (start 143.236396 83.85) (end 157.513604 83.85) (width 0.25) (layer "F.Cu") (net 4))
 (segment (start 146.978604 63.331) (end 146.38 63.929604) (width 0.25) (layer "F.Cu") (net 4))
 (segment (start 151.565 57.095) (end 152.89 58.42) (width 0.25) (layer "F.Cu") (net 4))
 (segment (start 151.5531 70.6) (end 151.5531 70.951) (width 0.25) (layer "F.Cu") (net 4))
 (segment (start 159.054 69.07) (end 161.885 69.07) (width 0.25) (layer "F.Cu") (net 4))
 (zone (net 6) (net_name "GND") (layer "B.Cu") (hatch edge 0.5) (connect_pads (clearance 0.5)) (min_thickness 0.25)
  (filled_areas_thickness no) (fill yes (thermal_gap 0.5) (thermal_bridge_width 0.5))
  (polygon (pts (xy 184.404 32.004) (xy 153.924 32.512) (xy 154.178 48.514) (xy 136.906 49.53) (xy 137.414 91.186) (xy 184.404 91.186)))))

